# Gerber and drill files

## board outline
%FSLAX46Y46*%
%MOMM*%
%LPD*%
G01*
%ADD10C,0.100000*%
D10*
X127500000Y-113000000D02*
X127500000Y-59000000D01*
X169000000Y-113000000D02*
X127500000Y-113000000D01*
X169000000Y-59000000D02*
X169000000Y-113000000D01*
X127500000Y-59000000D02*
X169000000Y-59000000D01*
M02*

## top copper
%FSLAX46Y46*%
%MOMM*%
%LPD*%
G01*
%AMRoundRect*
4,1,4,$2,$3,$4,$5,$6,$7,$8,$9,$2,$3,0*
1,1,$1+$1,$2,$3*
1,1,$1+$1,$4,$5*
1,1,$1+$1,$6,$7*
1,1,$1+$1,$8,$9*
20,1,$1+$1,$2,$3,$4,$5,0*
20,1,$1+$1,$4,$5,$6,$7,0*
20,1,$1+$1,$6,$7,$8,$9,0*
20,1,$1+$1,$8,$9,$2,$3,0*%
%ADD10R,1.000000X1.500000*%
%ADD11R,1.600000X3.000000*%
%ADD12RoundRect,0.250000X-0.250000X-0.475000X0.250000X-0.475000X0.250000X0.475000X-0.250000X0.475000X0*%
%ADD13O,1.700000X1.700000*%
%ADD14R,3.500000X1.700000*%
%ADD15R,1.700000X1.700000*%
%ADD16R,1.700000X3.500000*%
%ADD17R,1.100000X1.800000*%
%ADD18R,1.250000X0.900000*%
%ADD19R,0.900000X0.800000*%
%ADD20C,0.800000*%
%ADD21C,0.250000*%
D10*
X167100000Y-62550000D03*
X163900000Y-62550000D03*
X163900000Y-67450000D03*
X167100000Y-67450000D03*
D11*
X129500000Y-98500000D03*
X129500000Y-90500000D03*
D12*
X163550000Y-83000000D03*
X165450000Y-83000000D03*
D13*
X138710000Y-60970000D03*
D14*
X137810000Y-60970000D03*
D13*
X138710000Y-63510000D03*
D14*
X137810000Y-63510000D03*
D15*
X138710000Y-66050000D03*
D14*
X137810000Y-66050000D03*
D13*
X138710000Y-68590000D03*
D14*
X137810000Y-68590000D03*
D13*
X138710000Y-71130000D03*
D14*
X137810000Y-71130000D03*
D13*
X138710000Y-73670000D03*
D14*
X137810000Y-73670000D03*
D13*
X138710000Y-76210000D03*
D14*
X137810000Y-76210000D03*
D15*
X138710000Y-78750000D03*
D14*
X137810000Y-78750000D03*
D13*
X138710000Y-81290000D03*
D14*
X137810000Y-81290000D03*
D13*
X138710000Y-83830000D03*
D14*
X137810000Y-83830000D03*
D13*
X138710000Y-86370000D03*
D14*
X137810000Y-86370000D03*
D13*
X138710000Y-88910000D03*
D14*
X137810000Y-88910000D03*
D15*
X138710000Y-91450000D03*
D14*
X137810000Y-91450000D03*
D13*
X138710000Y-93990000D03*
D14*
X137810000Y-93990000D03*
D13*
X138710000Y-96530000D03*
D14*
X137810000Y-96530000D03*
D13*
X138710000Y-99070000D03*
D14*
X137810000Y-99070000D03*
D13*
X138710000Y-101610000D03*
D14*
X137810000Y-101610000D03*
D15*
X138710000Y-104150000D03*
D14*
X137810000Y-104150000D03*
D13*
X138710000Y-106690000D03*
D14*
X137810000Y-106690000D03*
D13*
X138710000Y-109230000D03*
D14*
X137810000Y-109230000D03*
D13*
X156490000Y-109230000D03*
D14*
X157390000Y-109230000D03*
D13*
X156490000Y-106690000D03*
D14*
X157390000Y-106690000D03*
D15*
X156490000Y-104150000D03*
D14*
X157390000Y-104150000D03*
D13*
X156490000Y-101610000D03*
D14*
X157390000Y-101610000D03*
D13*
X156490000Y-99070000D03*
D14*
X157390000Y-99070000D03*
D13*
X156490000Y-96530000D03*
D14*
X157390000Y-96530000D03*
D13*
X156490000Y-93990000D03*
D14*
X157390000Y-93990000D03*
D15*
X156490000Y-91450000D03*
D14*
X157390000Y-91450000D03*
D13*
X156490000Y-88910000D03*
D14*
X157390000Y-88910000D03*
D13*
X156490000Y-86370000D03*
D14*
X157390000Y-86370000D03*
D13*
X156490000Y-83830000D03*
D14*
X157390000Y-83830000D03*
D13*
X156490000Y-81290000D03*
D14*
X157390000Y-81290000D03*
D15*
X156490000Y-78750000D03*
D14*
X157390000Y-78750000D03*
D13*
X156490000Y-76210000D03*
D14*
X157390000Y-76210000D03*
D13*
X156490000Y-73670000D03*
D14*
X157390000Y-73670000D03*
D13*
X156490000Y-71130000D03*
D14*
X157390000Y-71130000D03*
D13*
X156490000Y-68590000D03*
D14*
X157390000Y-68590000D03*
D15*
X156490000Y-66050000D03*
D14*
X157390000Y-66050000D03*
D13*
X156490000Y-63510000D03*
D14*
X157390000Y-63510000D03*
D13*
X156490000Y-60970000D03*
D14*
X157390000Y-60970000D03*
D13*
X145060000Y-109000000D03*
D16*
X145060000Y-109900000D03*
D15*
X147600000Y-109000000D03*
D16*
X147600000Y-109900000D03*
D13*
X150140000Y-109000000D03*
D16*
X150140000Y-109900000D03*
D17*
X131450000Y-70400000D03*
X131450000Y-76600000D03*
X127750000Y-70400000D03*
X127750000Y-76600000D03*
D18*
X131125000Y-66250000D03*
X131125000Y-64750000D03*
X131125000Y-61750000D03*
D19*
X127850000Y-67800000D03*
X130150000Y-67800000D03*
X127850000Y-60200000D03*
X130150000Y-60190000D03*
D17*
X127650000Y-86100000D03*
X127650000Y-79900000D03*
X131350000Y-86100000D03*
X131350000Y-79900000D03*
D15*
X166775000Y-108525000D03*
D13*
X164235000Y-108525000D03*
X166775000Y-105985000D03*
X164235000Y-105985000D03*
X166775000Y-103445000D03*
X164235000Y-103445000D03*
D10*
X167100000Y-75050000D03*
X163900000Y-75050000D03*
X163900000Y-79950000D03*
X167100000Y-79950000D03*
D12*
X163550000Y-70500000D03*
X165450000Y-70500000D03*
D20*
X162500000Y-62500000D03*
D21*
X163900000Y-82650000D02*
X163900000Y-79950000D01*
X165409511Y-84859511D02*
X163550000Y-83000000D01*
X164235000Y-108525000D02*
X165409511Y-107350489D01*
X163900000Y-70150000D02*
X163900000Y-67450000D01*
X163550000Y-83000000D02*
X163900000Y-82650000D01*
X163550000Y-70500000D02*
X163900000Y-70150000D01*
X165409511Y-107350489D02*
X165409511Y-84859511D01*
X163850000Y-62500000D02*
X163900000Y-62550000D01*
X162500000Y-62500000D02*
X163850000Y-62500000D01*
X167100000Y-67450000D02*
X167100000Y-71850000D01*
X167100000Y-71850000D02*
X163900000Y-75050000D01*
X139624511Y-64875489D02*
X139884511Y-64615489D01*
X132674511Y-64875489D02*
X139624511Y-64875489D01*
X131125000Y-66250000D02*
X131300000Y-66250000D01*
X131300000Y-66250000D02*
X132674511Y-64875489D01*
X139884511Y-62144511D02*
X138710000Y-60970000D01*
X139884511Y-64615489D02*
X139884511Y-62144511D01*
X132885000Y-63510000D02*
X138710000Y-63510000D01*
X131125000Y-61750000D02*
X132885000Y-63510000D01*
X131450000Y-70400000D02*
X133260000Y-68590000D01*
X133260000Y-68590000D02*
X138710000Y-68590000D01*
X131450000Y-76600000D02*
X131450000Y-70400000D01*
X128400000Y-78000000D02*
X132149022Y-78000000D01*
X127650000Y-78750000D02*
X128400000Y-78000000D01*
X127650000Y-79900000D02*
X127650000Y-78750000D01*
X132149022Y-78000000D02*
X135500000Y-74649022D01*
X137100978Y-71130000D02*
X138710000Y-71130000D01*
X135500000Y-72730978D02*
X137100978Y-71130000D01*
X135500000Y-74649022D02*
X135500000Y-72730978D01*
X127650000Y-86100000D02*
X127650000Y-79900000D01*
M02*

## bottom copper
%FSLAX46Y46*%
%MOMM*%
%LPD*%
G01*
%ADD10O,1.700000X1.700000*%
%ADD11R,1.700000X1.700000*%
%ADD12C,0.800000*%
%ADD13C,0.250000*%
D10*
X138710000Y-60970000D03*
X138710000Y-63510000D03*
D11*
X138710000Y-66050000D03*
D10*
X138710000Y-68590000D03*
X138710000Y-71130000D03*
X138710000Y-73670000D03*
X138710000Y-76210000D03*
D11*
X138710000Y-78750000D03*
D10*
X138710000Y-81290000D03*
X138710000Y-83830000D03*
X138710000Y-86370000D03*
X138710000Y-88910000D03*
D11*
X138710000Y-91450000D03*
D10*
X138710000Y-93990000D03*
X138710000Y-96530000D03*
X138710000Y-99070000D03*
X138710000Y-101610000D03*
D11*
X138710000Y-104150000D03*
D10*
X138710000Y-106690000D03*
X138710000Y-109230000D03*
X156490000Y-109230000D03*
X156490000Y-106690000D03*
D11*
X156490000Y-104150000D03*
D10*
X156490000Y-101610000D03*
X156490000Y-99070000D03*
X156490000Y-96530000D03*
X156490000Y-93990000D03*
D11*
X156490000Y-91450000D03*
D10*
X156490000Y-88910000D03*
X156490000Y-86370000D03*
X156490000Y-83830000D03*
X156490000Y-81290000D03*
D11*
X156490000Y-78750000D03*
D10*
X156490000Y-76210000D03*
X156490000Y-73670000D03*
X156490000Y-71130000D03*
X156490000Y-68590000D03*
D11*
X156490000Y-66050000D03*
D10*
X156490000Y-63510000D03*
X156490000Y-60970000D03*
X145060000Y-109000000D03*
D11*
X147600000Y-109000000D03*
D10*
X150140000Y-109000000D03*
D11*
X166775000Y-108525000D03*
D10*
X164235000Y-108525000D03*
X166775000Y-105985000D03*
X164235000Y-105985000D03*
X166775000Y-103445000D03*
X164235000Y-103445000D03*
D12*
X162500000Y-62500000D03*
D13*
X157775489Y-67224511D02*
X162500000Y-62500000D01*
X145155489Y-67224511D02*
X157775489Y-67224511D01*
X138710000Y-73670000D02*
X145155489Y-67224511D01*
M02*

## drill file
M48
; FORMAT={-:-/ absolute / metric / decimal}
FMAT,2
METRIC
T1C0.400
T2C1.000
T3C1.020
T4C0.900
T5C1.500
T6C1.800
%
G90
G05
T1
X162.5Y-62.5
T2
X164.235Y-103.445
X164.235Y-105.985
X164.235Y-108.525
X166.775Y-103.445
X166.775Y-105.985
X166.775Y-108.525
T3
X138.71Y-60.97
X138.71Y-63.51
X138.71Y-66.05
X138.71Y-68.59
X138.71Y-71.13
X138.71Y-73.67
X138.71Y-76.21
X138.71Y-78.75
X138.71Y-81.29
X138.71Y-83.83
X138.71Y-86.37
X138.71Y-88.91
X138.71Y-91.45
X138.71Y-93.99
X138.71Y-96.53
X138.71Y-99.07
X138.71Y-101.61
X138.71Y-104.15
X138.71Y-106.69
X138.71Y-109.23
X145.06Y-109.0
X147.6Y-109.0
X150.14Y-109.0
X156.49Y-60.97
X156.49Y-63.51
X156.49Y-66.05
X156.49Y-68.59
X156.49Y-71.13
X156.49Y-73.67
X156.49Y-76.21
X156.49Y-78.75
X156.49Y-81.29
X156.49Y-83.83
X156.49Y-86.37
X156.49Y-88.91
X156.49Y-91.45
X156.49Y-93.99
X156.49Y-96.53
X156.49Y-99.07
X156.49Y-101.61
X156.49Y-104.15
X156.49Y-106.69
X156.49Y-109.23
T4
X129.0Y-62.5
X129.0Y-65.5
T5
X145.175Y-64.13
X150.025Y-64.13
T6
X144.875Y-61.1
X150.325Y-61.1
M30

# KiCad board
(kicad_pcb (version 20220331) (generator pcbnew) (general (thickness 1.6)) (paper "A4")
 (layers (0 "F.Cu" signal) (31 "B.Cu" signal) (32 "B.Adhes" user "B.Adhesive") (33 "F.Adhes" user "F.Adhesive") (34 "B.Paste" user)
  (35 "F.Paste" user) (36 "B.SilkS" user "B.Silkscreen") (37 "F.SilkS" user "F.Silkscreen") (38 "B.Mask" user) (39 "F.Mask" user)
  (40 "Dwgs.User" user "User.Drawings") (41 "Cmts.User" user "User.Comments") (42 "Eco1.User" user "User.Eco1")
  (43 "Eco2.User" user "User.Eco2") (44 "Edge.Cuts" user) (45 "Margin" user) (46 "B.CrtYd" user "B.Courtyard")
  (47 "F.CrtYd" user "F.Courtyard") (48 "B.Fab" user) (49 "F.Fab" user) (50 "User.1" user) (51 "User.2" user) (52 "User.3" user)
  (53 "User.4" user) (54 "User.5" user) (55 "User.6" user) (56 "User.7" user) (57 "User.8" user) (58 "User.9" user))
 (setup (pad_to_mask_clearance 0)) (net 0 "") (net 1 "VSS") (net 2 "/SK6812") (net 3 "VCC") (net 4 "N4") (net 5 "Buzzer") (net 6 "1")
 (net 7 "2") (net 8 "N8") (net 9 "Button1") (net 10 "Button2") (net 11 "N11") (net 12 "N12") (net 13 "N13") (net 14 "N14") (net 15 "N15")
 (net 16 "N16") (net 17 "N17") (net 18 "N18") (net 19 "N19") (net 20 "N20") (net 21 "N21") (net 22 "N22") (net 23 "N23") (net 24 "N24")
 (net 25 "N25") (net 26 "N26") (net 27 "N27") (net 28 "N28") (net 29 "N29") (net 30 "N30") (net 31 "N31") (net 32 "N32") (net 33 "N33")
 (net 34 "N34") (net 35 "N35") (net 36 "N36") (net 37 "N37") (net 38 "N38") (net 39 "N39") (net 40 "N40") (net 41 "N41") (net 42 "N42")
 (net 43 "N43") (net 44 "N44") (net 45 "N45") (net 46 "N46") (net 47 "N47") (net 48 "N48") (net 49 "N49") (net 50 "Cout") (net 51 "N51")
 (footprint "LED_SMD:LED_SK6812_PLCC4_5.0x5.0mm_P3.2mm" (layer "F.Cu") (at 165.5 65 90)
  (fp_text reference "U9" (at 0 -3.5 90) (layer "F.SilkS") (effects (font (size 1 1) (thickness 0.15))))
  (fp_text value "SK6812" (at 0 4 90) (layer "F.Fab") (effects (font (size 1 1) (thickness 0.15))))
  (pad "1" smd rect (at 2.45 1.6 90) (size 1.5 1) (layers "F.Cu" "F.Paste" "F.Mask") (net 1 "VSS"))
  (pad "2" smd rect (at 2.45 -1.6 90) (size 1.5 1) (layers "F.Cu" "F.Paste" "F.Mask") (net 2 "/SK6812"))
  (pad "3" smd rect (at -2.45 -1.6 90) (size 1.5 1) (layers "F.Cu" "F.Paste" "F.Mask") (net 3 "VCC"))
  (pad "4" smd rect (at -2.45 1.6 90) (size 1.5 1) (layers "F.Cu" "F.Paste" "F.Mask") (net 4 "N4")))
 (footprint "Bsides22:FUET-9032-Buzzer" (layer "F.Cu") (at 129.5 98.5 90)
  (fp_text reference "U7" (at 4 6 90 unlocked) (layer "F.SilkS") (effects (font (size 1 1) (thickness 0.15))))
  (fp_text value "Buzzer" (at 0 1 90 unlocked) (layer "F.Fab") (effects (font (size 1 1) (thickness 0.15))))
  (pad "1" smd rect (at 0 0 90) (size 3 1.6) (layers "F.Cu" "F.Paste" "F.Mask") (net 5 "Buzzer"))
  (pad "2" smd rect (at 8 0 90) (size 3 1.6) (layers "F.Cu" "F.Paste" "F.Mask") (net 1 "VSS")))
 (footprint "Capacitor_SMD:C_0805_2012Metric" (layer "F.Cu") (at 164.5 83)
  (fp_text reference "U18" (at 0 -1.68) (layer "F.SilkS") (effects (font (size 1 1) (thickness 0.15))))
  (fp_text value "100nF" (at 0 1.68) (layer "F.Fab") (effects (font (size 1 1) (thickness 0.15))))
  (pad "1" smd roundrect (at -0.95 0) (size 1 1.45) (layers "F.Cu" "F.Paste" "F.Mask") (roundrect_rratio 0.25) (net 3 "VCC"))
  (pad "2" smd roundrect (at 0.95 0) (size 1 1.45) (layers "F.Cu" "F.Paste" "F.Mask") (roundrect_rratio 0.25) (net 1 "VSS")))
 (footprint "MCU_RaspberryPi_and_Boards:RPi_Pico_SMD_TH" (layer "F.Cu") (at 147.6 85.1)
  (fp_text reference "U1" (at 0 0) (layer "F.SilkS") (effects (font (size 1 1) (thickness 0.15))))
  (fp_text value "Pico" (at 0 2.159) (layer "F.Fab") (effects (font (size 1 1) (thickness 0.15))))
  (pad "" np_thru_hole oval (at -2.725 -24) (size 1.8 1.8) (drill 1.8) (layers *.Cu *.Mask))
  (pad "" np_thru_hole oval (at -2.425 -20.97) (size 1.5 1.5) (drill 1.5) (layers *.Cu *.Mask))
  (pad "" np_thru_hole oval (at 2.425 -20.97) (size 1.5 1.5) (drill 1.5) (layers *.Cu *.Mask))
  (pad "" np_thru_hole oval (at 2.725 -24) (size 1.8 1.8) (drill 1.8) (layers *.Cu *.Mask))
  (pad "1" thru_hole oval (at -8.89 -24.13) (size 1.7 1.7) (drill 1.02) (layers *.Cu *.Mask) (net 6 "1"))
  (pad "1" smd rect (at -8.89 -24.13) (size 3.5 1.7) (drill (offset -0.9 0)) (layers "F.Cu" "F.Mask") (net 6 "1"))
  (pad "2" thru_hole oval (at -8.89 -21.59) (size 1.7 1.7) (drill 1.02) (layers *.Cu *.Mask) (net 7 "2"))
  (pad "2" smd rect (at -8.89 -21.59) (size 3.5 1.7) (drill (offset -0.9 0)) (layers "F.Cu" "F.Mask") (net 7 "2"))
  (pad "3" thru_hole rect (at -8.89 -19.05) (size 1.7 1.7) (drill 1.02) (layers *.Cu *.Mask) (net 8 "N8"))
  (pad "3" smd rect (at -8.89 -19.05) (size 3.5 1.7) (drill (offset -0.9 0)) (layers "F.Cu" "F.Mask") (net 8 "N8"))
  (pad "4" thru_hole oval (at -8.89 -16.51) (size 1.7 1.7) (drill 1.02) (layers *.Cu *.Mask) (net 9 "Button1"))
  (pad "4" smd rect (at -8.89 -16.51) (size 3.5 1.7) (drill (offset -0.9 0)) (layers "F.Cu" "F.Mask") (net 9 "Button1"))
  (pad "5" thru_hole oval (at -8.89 -13.97) (size 1.7 1.7) (drill 1.02) (layers *.Cu *.Mask) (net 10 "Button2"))
  (pad "5" smd rect (at -8.89 -13.97) (size 3.5 1.7) (drill (offset -0.9 0)) (layers "F.Cu" "F.Mask") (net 10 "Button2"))
  (pad "6" thru_hole oval (at -8.89 -11.43) (size 1.7 1.7) (drill 1.02) (layers *.Cu *.Mask) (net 2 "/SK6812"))
  (pad "6" smd rect (at -8.89 -11.43) (size 3.5 1.7) (drill (offset -0.9 0)) (layers "F.Cu" "F.Mask") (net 2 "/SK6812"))
  (pad "7" thru_hole oval (at -8.89 -8.89) (size 1.7 1.7) (drill 1.02) (layers *.Cu *.Mask) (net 5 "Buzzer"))
  (pad "7" smd rect (at -8.89 -8.89) (size 3.5 1.7) (drill (offset -0.9 0)) (layers "F.Cu" "F.Mask") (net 5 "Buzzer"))
  (pad "8" thru_hole rect (at -8.89 -6.35) (size 1.7 1.7) (drill 1.02) (layers *.Cu *.Mask) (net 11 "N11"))
  (pad "8" smd rect (at -8.89 -6.35) (size 3.5 1.7) (drill (offset -0.9 0)) (layers "F.Cu" "F.Mask") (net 11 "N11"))
  (pad "9" thru_hole oval (at -8.89 -3.81) (size 1.7 1.7) (drill 1.02) (layers *.Cu *.Mask) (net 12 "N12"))
  (pad "9" smd rect (at -8.89 -3.81) (size 3.5 1.7) (drill (offset -0.9 0)) (layers "F.Cu" "F.Mask") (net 12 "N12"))
  (pad "10" thru_hole oval (at -8.89 -1.27) (size 1.7 1.7) (drill 1.02) (layers *.Cu *.Mask) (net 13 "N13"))
  (pad "10" smd rect (at -8.89 -1.27) (size 3.5 1.7) (drill (offset -0.9 0)) (layers "F.Cu" "F.Mask") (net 13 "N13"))
  (pad "11" thru_hole oval (at -8.89 1.27) (size 1.7 1.7) (drill 1.02) (layers *.Cu *.Mask) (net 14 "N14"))
  (pad "11" smd rect (at -8.89 1.27) (size 3.5 1.7) (drill (offset -0.9 0)) (layers "F.Cu" "F.Mask") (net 14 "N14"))
  (pad "12" thru_hole oval (at -8.89 3.81) (size 1.7 1.7) (drill 1.02) (layers *.Cu *.Mask) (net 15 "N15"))
  (pad "12" smd rect (at -8.89 3.81) (size 3.5 1.7) (drill (offset -0.9 0)) (layers "F.Cu" "F.Mask") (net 15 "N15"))
  (pad "13" thru_hole rect (at -8.89 6.35) (size 1.7 1.7) (drill 1.02) (layers *.Cu *.Mask) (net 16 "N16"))
  (pad "13" smd rect (at -8.89 6.35) (size 3.5 1.7) (drill (offset -0.9 0)) (layers "F.Cu" "F.Mask") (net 16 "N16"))
  (pad "14" thru_hole oval (at -8.89 8.89) (size 1.7 1.7) (drill 1.02) (layers *.Cu *.Mask) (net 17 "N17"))
  (pad "14" smd rect (at -8.89 8.89) (size 3.5 1.7) (drill (offset -0.9 0)) (layers "F.Cu" "F.Mask") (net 17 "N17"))
  (pad "15" thru_hole oval (at -8.89 11.43) (size 1.7 1.7) (drill 1.02) (layers *.Cu *.Mask) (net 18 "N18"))
  (pad "15" smd rect (at -8.89 11.43) (size 3.5 1.7) (drill (offset -0.9 0)) (layers "F.Cu" "F.Mask") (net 18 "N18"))
  (pad "16" thru_hole oval (at -8.89 13.97) (size 1.7 1.7) (drill 1.02) (layers *.Cu *.Mask) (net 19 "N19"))
  (pad "16" smd rect (at -8.89 13.97) (size 3.5 1.7) (drill (offset -0.9 0)) (layers "F.Cu" "F.Mask") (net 19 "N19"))
  (pad "17" thru_hole oval (at -8.89 16.51) (size 1.7 1.7) (drill 1.02) (layers *.Cu *.Mask) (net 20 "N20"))
  (pad "17" smd rect (at -8.89 16.51) (size 3.5 1.7) (drill (offset -0.9 0)) (layers "F.Cu" "F.Mask") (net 20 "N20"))
  (pad "18" thru_hole rect (at -8.89 19.05) (size 1.7 1.7) (drill 1.02) (layers *.Cu *.Mask) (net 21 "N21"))
  (pad "18" smd rect (at -8.89 19.05) (size 3.5 1.7) (drill (offset -0.9 0)) (layers "F.Cu" "F.Mask") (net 21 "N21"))
  (pad "19" thru_hole oval (at -8.89 21.59) (size 1.7 1.7) (drill 1.02) (layers *.Cu *.Mask) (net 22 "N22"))
  (pad "19" smd rect (at -8.89 21.59) (size 3.5 1.7) (drill (offset -0.9 0)) (layers "F.Cu" "F.Mask") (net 22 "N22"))
  (pad "20" thru_hole oval (at -8.89 24.13) (size 1.7 1.7) (drill 1.02) (layers *.Cu *.Mask) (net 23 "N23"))
  (pad "20" smd rect (at -8.89 24.13) (size 3.5 1.7) (drill (offset -0.9 0)) (layers "F.Cu" "F.Mask") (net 23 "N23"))
  (pad "21" thru_hole oval (at 8.89 24.13) (size 1.7 1.7) (drill 1.02) (layers *.Cu *.Mask) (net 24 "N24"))
  (pad "21" smd rect (at 8.89 24.13) (size 3.5 1.7) (drill (offset 0.9 0)) (layers "F.Cu" "F.Mask") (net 24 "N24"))
  (pad "22" thru_hole oval (at 8.89 21.59) (size 1.7 1.7) (drill 1.02) (layers *.Cu *.Mask) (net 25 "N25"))
  (pad "22" smd rect (at 8.89 21.59) (size 3.5 1.7) (drill (offset 0.9 0)) (layers "F.Cu" "F.Mask") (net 25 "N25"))
  (pad "23" thru_hole rect (at 8.89 19.05) (size 1.7 1.7) (drill 1.02) (layers *.Cu *.Mask) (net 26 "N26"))
  (pad "23" smd rect (at 8.89 19.05) (size 3.5 1.7) (drill (offset 0.9 0)) (layers "F.Cu" "F.Mask") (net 26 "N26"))
  (pad "24" thru_hole oval (at 8.89 16.51) (size 1.7 1.7) (drill 1.02) (layers *.Cu *.Mask) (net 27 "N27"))
  (pad "24" smd rect (at 8.89 16.51) (size 3.5 1.7) (drill (offset 0.9 0)) (layers "F.Cu" "F.Mask") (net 27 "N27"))
  (pad "25" thru_hole oval (at 8.89 13.97) (size 1.7 1.7) (drill 1.02) (layers *.Cu *.Mask) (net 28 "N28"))
  (pad "25" smd rect (at 8.89 13.97) (size 3.5 1.7) (drill (offset 0.9 0)) (layers "F.Cu" "F.Mask") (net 28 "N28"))
  (pad "26" thru_hole oval (at 8.89 11.43) (size 1.7 1.7) (drill 1.02) (layers *.Cu *.Mask) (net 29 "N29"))
  (pad "26" smd rect (at 8.89 11.43) (size 3.5 1.7) (drill (offset 0.9 0)) (layers "F.Cu" "F.Mask") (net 29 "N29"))
  (pad "27" thru_hole oval (at 8.89 8.89) (size 1.7 1.7) (drill 1.02) (layers *.Cu *.Mask) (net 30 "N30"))
  (pad "27" smd rect (at 8.89 8.89) (size 3.5 1.7) (drill (offset 0.9 0)) (layers "F.Cu" "F.Mask") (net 30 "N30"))
  (pad "28" thru_hole rect (at 8.89 6.35) (size 1.7 1.7) (drill 1.02) (layers *.Cu *.Mask) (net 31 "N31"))
  (pad "28" smd rect (at 8.89 6.35) (size 3.5 1.7) (drill (offset 0.9 0)) (layers "F.Cu" "F.Mask") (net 31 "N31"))
  (pad "29" thru_hole oval (at 8.89 3.81) (size 1.7 1.7) (drill 1.02) (layers *.Cu *.Mask) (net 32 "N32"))
  (pad "29" smd rect (at 8.89 3.81) (size 3.5 1.7) (drill (offset 0.9 0)) (layers "F.Cu" "F.Mask") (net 32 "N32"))
  (pad "30" thru_hole oval (at 8.89 1.27) (size 1.7 1.7) (drill 1.02) (layers *.Cu *.Mask) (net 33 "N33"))
  (pad "30" smd rect (at 8.89 1.27) (size 3.5 1.7) (drill (offset 0.9 0)) (layers "F.Cu" "F.Mask") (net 33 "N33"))
  (pad "31" thru_hole oval (at 8.89 -1.27) (size 1.7 1.7) (drill 1.02) (layers *.Cu *.Mask) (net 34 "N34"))
  (pad "31" smd rect (at 8.89 -1.27) (size 3.5 1.7) (drill (offset 0.9 0)) (layers "F.Cu" "F.Mask") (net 34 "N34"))
  (pad "32" thru_hole oval (at 8.89 -3.81) (size 1.7 1.7) (drill 1.02) (layers *.Cu *.Mask) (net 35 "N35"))
  (pad "32" smd rect (at 8.89 -3.81) (size 3.5 1.7) (drill (offset 0.9 0)) (layers "F.Cu" "F.Mask") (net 35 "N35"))
  (pad "33" thru_hole rect (at 8.89 -6.35) (size 1.7 1.7) (drill 1.02) (layers *.Cu *.Mask) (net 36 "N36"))
  (pad "33" smd rect (at 8.89 -6.35) (size 3.5 1.7) (drill (offset 0.9 0)) (layers "F.Cu" "F.Mask") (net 36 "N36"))
  (pad "34" thru_hole oval (at 8.89 -8.89) (size 1.7 1.7) (drill 1.02) (layers *.Cu *.Mask) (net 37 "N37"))
  (pad "34" smd rect (at 8.89 -8.89) (size 3.5 1.7) (drill (offset 0.9 0)) (layers "F.Cu" "F.Mask") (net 37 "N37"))
  (pad "35" thru_hole oval (at 8.89 -11.43) (size 1.7 1.7) (drill 1.02) (layers *.Cu *.Mask) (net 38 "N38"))
  (pad "35" smd rect (at 8.89 -11.43) (size 3.5 1.7) (drill (offset 0.9 0)) (layers "F.Cu" "F.Mask") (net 38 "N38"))
  (pad "36" thru_hole oval (at 8.89 -13.97) (size 1.7 1.7) (drill 1.02) (layers *.Cu *.Mask) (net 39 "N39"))
  (pad "36" smd rect (at 8.89 -13.97) (size 3.5 1.7) (drill (offset 0.9 0)) (layers "F.Cu" "F.Mask") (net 39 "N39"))
  (pad "37" thru_hole oval (at 8.89 -16.51) (size 1.7 1.7) (drill 1.02) (layers *.Cu *.Mask) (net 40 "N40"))
  (pad "37" smd rect (at 8.89 -16.51) (size 3.5 1.7) (drill (offset 0.9 0)) (layers "F.Cu" "F.Mask") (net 40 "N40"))
  (pad "38" thru_hole rect (at 8.89 -19.05) (size 1.7 1.7) (drill 1.02) (layers *.Cu *.Mask) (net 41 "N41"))
  (pad "38" smd rect (at 8.89 -19.05) (size 3.5 1.7) (drill (offset 0.9 0)) (layers "F.Cu" "F.Mask") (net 41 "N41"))
  (pad "39" thru_hole oval (at 8.89 -21.59) (size 1.7 1.7) (drill 1.02) (layers *.Cu *.Mask) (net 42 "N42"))
  (pad "39" smd rect (at 8.89 -21.59) (size 3.5 1.7) (drill (offset 0.9 0)) (layers "F.Cu" "F.Mask") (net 42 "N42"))
  (pad "40" thru_hole oval (at 8.89 -24.13) (size 1.7 1.7) (drill 1.02) (layers *.Cu *.Mask) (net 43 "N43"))
  (pad "40" smd rect (at 8.89 -24.13) (size 3.5 1.7) (drill (offset 0.9 0)) (layers "F.Cu" "F.Mask") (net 43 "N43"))
  (pad "41" thru_hole oval (at -2.54 23.9) (size 1.7 1.7) (drill 1.02) (layers *.Cu *.Mask) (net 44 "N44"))
  (pad "41" smd rect (at -2.54 23.9 90) (size 3.5 1.7) (drill (offset -0.9 0)) (layers "F.Cu" "F.Mask") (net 44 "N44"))
  (pad "42" thru_hole rect (at 0 23.9) (size 1.7 1.7) (drill 1.02) (layers *.Cu *.Mask) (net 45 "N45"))
  (pad "42" smd rect (at 0 23.9 90) (size 3.5 1.7) (drill (offset -0.9 0)) (layers "F.Cu" "F.Mask") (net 45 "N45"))
  (pad "43" thru_hole oval (at 2.54 23.9) (size 1.7 1.7) (drill 1.02) (layers *.Cu *.Mask) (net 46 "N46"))
  (pad "43" smd rect (at 2.54 23.9 90) (size 3.5 1.7) (drill (offset -0.9 0)) (layers "F.Cu" "F.Mask") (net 46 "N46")))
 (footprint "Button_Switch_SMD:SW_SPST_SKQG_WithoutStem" (layer "F.Cu") (at 129.6 73.5 -90)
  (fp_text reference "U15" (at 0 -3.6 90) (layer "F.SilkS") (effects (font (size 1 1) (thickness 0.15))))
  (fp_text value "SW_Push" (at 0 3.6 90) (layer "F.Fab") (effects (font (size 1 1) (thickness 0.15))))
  (pad "1" smd rect (at -3.1 -1.85 270) (size 1.8 1.1) (layers "F.Cu" "F.Paste" "F.Mask") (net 9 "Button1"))
  (pad "1" smd rect (at 3.1 -1.85 270) (size 1.8 1.1) (layers "F.Cu" "F.Paste" "F.Mask") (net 9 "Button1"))
  (pad "2" smd rect (at -3.1 1.85 270) (size 1.8 1.1) (layers "F.Cu" "F.Paste" "F.Mask") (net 1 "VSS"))
  (pad "2" smd rect (at 3.1 1.85 270) (size 1.8 1.1) (layers "F.Cu" "F.Paste" "F.Mask") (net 1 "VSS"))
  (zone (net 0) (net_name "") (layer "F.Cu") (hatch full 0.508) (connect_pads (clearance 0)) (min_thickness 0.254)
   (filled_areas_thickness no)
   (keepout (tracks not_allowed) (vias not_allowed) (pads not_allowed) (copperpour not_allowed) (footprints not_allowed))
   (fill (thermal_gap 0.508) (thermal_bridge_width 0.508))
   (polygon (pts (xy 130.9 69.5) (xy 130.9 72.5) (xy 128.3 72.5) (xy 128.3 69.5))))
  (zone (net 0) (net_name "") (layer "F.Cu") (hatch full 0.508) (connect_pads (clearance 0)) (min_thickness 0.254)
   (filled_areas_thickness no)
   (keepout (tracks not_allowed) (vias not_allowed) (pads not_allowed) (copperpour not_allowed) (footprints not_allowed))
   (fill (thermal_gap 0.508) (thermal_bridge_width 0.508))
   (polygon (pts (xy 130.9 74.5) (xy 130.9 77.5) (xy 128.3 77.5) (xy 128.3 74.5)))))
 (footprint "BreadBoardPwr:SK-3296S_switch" (layer "F.Cu") (at 129 64 90)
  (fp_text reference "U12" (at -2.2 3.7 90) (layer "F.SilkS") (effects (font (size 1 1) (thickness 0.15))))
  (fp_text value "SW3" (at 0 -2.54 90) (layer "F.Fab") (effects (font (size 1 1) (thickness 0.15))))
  (pad "" np_thru_hole circle locked (at -1.5 0 90) (size 0.9 0.9) (drill 0.9) (layers *.Cu *.Mask))
  (pad "" np_thru_hole circle locked (at 1.5 0 90) (size 0.9 0.9) (drill 0.9) (layers *.Cu *.Mask))
  (pad "1" smd rect locked (at -2.25 2.125 90) (size 0.9 1.25) (layers "F.Cu" "F.Paste" "F.Mask") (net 6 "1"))
  (pad "2" smd rect locked (at -0.75 2.125 90) (size 0.9 1.25) (layers "F.Cu" "F.Paste" "F.Mask") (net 1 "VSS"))
  (pad "3" smd rect locked (at 2.25 2.125 90) (size 0.9 1.25) (layers "F.Cu" "F.Paste" "F.Mask") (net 7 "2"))
  (pad "4" smd rect locked (at -3.8 -1.15 90) (size 0.8 0.9) (layers "F.Cu" "F.Paste" "F.Mask"))
  (pad "4" smd rect locked (at -3.8 1.15 90) (size 0.8 0.9) (layers "F.Cu" "F.Paste" "F.Mask"))
  (pad "4" smd rect locked (at 3.8 -1.15 90) (size 0.8 0.9) (layers "F.Cu" "F.Paste" "F.Mask"))
  (pad "4" smd rect locked (at 3.81 1.15 90) (size 0.8 0.9) (layers "F.Cu" "F.Paste" "F.Mask")))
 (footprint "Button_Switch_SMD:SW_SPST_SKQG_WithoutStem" (layer "F.Cu") (at 129.5 83 90)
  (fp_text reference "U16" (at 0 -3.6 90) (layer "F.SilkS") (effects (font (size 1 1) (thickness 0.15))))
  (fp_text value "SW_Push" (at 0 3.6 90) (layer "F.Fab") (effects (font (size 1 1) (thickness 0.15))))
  (pad "1" smd rect (at -3.1 -1.85 90) (size 1.8 1.1) (layers "F.Cu" "F.Paste" "F.Mask") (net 10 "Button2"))
  (pad "1" smd rect (at 3.1 -1.85 90) (size 1.8 1.1) (layers "F.Cu" "F.Paste" "F.Mask") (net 10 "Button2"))
  (pad "2" smd rect (at -3.1 1.85 90) (size 1.8 1.1) (layers "F.Cu" "F.Paste" "F.Mask") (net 1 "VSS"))
  (pad "2" smd rect (at 3.1 1.85 90) (size 1.8 1.1) (layers "F.Cu" "F.Paste" "F.Mask") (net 1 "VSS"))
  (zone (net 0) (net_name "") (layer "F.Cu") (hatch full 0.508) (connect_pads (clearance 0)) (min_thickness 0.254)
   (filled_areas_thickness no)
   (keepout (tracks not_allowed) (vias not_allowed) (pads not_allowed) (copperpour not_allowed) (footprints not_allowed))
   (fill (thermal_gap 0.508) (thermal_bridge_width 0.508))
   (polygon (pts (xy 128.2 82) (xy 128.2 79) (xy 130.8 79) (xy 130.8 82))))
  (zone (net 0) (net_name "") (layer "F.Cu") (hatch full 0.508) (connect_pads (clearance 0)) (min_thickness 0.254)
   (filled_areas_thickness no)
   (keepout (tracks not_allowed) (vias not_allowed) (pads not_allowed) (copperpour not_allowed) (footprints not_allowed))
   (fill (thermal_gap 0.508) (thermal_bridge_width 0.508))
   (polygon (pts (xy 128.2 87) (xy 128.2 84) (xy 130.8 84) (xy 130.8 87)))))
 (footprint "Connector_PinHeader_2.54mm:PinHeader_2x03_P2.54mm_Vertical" (layer "F.Cu") (at 166.775 108.525 180)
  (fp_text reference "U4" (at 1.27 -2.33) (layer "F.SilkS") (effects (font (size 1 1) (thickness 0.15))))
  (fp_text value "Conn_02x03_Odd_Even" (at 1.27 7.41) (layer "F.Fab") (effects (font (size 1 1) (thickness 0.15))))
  (pad "1" thru_hole rect (at 0 0 180) (size 1.7 1.7) (drill 1) (layers *.Cu *.Mask) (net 1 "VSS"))
  (pad "2" thru_hole oval (at 2.54 0 180) (size 1.7 1.7) (drill 1) (layers *.Cu *.Mask) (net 3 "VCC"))
  (pad "3" thru_hole oval (at 0 2.54 180) (size 1.7 1.7) (drill 1) (layers *.Cu *.Mask) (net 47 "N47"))
  (pad "4" thru_hole oval (at 2.54 2.54 180) (size 1.7 1.7) (drill 1) (layers *.Cu *.Mask) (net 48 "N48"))
  (pad "5" thru_hole oval (at 0 5.08 180) (size 1.7 1.7) (drill 1) (layers *.Cu *.Mask) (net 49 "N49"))
  (pad "6" thru_hole oval (at 2.54 5.08 180) (size 1.7 1.7) (drill 1) (layers *.Cu *.Mask) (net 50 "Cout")))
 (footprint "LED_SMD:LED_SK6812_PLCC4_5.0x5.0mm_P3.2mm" (layer "F.Cu") (at 165.5 77.5 90)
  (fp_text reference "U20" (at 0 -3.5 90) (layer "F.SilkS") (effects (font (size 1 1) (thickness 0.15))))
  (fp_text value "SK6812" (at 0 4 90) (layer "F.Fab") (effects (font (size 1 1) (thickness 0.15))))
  (pad "1" smd rect (at 2.45 1.6 90) (size 1.5 1) (layers "F.Cu" "F.Paste" "F.Mask") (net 1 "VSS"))
  (pad "2" smd rect (at 2.45 -1.6 90) (size 1.5 1) (layers "F.Cu" "F.Paste" "F.Mask") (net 4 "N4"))
  (pad "3" smd rect (at -2.45 -1.6 90) (size 1.5 1) (layers "F.Cu" "F.Paste" "F.Mask") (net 3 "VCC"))
  (pad "4" smd rect (at -2.45 1.6 90) (size 1.5 1) (layers "F.Cu" "F.Paste" "F.Mask") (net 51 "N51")))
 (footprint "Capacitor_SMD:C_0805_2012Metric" (layer "F.Cu") (at 164.5 70.5)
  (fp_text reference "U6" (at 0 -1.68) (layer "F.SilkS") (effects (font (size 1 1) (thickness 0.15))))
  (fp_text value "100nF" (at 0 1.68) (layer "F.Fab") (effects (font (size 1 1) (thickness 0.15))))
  (pad "1" smd roundrect (at -0.95 0) (size 1 1.45) (layers "F.Cu" "F.Paste" "F.Mask") (roundrect_rratio 0.25) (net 3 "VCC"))
  (pad "2" smd roundrect (at 0.95 0) (size 1 1.45) (layers "F.Cu" "F.Paste" "F.Mask") (roundrect_rratio 0.25) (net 1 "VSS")))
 (gr_line (start 127.5 113) (end 127.5 59) (stroke (width 0.1) (type default)) (layer "Edge.Cuts"))
 (gr_line (start 169 113) (end 127.5 113) (stroke (width 0.1) (type default)) (layer "Edge.Cuts"))
 (gr_line (start 169 59) (end 169 113) (stroke (width 0.1) (type default)) (layer "Edge.Cuts"))
 (gr_line (start 127.5 59) (end 169 59) (stroke (width 0.1) (type default)) (layer "Edge.Cuts"))
 (segment (start 163.9 82.65) (end 163.9 79.95) (width 0.25) (layer "F.Cu") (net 3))
 (segment (start 165.409511 84.859511) (end 163.55 83) (width 0.25) (layer "F.Cu") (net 3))
 (segment (start 164.235 108.525) (end 165.409511 107.350489) (width 0.25) (layer "F.Cu") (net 3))
 (segment (start 163.9 70.15) (end 163.9 67.45) (width 0.25) (layer "F.Cu") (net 3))
 (segment (start 163.55 83) (end 163.9 82.65) (width 0.25) (layer "F.Cu") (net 3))
 (segment (start 163.55 70.5) (end 163.9 70.15) (width 0.25) (layer "F.Cu") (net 3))
 (segment (start 165.409511 107.350489) (end 165.409511 84.859511) (width 0.25) (layer "F.Cu") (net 3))
 (segment (start 163.85 62.5) (end 163.9 62.55) (width 0.25) (layer "F.Cu") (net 2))
 (segment (start 162.5 62.5) (end 163.85 62.5) (width 0.25) (layer "F.Cu") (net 2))
 (via (at 162.5 62.5) (size 0.8) (drill 0.4) (layers "F.Cu" "B.Cu") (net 2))
 (segment (start 157.775489 67.224511) (end 162.5 62.5) (width 0.25) (layer "B.Cu") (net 2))
 (segment (start 145.155489 67.224511) (end 157.775489 67.224511) (width 0.25) (layer "B.Cu") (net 2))
 (segment (start 138.71 73.67) (end 145.155489 67.224511) (width 0.25) (layer "B.Cu") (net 2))
 (segment (start 167.1 67.45) (end 167.1 71.85) (width 0.25) (layer "F.Cu") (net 4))
 (segment (start 167.1 71.85) (end 163.9 75.05) (width 0.25) (layer "F.Cu") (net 4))
 (segment (start 139.624511 64.875489) (end 139.884511 64.615489) (width 0.25) (layer "F.Cu") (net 6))
 (segment (start 132.674511 64.875489) (end 139.624511 64.875489) (width 0.25) (layer "F.Cu") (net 6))
 (segment (start 131.125 66.25) (end 131.3 66.25) (width 0.25) (layer "F.Cu") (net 6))
 (segment (start 131.3 66.25) (end 132.674511 64.875489) (width 0.25) (layer "F.Cu") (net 6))
 (segment (start 139.884511 62.144511) (end 138.71 60.97) (width 0.25) (layer "F.Cu") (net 6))
 (segment (start 139.884511 64.615489) (end 139.884511 62.144511) (width 0.25) (layer "F.Cu") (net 6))
 (segment (start 132.885 63.51) (end 138.71 63.51) (width 0.25) (layer "F.Cu") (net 7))
 (segment (start 131.125 61.75) (end 132.885 63.51) (width 0.25) (layer "F.Cu") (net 7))
 (segment (start 131.45 70.4) (end 133.26 68.59) (width 0.25) (layer "F.Cu") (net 9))
 (segment (start 133.26 68.59) (end 138.71 68.59) (width 0.25) (layer "F.Cu") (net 9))
 (segment (start 131.45 76.6) (end 131.45 70.4) (width 0.25) (layer "F.Cu") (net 9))
 (segment (start 128.4 78) (end 132.149022 78) (width 0.25) (layer "F.Cu") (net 10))
 (segment (start 127.65 78.75) (end 128.4 78) (width 0.25) (layer "F.Cu") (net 10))
 (segment (start 127.65 79.9) (end 127.65 78.75) (width 0.25) (layer "F.Cu") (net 10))
 (segment (start 132.149022 78) (end 135.5 74.649022) (width 0.25) (layer "F.Cu") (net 10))
 (segment (start 137.100978 71.13) (end 138.71 71.13) (width 0.25) (layer "F.Cu") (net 10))
 (segment (start 135.5 72.730978) (end 137.100978 71.13) (width 0.25) (layer "F.Cu") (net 10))
 (segment (start 135.5 74.649022) (end 135.5 72.730978) (width 0.25) (layer "F.Cu") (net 10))
 (segment (start 127.65 86.1) (end 127.65 79.9) (width 0.25) (layer "F.Cu") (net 10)))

